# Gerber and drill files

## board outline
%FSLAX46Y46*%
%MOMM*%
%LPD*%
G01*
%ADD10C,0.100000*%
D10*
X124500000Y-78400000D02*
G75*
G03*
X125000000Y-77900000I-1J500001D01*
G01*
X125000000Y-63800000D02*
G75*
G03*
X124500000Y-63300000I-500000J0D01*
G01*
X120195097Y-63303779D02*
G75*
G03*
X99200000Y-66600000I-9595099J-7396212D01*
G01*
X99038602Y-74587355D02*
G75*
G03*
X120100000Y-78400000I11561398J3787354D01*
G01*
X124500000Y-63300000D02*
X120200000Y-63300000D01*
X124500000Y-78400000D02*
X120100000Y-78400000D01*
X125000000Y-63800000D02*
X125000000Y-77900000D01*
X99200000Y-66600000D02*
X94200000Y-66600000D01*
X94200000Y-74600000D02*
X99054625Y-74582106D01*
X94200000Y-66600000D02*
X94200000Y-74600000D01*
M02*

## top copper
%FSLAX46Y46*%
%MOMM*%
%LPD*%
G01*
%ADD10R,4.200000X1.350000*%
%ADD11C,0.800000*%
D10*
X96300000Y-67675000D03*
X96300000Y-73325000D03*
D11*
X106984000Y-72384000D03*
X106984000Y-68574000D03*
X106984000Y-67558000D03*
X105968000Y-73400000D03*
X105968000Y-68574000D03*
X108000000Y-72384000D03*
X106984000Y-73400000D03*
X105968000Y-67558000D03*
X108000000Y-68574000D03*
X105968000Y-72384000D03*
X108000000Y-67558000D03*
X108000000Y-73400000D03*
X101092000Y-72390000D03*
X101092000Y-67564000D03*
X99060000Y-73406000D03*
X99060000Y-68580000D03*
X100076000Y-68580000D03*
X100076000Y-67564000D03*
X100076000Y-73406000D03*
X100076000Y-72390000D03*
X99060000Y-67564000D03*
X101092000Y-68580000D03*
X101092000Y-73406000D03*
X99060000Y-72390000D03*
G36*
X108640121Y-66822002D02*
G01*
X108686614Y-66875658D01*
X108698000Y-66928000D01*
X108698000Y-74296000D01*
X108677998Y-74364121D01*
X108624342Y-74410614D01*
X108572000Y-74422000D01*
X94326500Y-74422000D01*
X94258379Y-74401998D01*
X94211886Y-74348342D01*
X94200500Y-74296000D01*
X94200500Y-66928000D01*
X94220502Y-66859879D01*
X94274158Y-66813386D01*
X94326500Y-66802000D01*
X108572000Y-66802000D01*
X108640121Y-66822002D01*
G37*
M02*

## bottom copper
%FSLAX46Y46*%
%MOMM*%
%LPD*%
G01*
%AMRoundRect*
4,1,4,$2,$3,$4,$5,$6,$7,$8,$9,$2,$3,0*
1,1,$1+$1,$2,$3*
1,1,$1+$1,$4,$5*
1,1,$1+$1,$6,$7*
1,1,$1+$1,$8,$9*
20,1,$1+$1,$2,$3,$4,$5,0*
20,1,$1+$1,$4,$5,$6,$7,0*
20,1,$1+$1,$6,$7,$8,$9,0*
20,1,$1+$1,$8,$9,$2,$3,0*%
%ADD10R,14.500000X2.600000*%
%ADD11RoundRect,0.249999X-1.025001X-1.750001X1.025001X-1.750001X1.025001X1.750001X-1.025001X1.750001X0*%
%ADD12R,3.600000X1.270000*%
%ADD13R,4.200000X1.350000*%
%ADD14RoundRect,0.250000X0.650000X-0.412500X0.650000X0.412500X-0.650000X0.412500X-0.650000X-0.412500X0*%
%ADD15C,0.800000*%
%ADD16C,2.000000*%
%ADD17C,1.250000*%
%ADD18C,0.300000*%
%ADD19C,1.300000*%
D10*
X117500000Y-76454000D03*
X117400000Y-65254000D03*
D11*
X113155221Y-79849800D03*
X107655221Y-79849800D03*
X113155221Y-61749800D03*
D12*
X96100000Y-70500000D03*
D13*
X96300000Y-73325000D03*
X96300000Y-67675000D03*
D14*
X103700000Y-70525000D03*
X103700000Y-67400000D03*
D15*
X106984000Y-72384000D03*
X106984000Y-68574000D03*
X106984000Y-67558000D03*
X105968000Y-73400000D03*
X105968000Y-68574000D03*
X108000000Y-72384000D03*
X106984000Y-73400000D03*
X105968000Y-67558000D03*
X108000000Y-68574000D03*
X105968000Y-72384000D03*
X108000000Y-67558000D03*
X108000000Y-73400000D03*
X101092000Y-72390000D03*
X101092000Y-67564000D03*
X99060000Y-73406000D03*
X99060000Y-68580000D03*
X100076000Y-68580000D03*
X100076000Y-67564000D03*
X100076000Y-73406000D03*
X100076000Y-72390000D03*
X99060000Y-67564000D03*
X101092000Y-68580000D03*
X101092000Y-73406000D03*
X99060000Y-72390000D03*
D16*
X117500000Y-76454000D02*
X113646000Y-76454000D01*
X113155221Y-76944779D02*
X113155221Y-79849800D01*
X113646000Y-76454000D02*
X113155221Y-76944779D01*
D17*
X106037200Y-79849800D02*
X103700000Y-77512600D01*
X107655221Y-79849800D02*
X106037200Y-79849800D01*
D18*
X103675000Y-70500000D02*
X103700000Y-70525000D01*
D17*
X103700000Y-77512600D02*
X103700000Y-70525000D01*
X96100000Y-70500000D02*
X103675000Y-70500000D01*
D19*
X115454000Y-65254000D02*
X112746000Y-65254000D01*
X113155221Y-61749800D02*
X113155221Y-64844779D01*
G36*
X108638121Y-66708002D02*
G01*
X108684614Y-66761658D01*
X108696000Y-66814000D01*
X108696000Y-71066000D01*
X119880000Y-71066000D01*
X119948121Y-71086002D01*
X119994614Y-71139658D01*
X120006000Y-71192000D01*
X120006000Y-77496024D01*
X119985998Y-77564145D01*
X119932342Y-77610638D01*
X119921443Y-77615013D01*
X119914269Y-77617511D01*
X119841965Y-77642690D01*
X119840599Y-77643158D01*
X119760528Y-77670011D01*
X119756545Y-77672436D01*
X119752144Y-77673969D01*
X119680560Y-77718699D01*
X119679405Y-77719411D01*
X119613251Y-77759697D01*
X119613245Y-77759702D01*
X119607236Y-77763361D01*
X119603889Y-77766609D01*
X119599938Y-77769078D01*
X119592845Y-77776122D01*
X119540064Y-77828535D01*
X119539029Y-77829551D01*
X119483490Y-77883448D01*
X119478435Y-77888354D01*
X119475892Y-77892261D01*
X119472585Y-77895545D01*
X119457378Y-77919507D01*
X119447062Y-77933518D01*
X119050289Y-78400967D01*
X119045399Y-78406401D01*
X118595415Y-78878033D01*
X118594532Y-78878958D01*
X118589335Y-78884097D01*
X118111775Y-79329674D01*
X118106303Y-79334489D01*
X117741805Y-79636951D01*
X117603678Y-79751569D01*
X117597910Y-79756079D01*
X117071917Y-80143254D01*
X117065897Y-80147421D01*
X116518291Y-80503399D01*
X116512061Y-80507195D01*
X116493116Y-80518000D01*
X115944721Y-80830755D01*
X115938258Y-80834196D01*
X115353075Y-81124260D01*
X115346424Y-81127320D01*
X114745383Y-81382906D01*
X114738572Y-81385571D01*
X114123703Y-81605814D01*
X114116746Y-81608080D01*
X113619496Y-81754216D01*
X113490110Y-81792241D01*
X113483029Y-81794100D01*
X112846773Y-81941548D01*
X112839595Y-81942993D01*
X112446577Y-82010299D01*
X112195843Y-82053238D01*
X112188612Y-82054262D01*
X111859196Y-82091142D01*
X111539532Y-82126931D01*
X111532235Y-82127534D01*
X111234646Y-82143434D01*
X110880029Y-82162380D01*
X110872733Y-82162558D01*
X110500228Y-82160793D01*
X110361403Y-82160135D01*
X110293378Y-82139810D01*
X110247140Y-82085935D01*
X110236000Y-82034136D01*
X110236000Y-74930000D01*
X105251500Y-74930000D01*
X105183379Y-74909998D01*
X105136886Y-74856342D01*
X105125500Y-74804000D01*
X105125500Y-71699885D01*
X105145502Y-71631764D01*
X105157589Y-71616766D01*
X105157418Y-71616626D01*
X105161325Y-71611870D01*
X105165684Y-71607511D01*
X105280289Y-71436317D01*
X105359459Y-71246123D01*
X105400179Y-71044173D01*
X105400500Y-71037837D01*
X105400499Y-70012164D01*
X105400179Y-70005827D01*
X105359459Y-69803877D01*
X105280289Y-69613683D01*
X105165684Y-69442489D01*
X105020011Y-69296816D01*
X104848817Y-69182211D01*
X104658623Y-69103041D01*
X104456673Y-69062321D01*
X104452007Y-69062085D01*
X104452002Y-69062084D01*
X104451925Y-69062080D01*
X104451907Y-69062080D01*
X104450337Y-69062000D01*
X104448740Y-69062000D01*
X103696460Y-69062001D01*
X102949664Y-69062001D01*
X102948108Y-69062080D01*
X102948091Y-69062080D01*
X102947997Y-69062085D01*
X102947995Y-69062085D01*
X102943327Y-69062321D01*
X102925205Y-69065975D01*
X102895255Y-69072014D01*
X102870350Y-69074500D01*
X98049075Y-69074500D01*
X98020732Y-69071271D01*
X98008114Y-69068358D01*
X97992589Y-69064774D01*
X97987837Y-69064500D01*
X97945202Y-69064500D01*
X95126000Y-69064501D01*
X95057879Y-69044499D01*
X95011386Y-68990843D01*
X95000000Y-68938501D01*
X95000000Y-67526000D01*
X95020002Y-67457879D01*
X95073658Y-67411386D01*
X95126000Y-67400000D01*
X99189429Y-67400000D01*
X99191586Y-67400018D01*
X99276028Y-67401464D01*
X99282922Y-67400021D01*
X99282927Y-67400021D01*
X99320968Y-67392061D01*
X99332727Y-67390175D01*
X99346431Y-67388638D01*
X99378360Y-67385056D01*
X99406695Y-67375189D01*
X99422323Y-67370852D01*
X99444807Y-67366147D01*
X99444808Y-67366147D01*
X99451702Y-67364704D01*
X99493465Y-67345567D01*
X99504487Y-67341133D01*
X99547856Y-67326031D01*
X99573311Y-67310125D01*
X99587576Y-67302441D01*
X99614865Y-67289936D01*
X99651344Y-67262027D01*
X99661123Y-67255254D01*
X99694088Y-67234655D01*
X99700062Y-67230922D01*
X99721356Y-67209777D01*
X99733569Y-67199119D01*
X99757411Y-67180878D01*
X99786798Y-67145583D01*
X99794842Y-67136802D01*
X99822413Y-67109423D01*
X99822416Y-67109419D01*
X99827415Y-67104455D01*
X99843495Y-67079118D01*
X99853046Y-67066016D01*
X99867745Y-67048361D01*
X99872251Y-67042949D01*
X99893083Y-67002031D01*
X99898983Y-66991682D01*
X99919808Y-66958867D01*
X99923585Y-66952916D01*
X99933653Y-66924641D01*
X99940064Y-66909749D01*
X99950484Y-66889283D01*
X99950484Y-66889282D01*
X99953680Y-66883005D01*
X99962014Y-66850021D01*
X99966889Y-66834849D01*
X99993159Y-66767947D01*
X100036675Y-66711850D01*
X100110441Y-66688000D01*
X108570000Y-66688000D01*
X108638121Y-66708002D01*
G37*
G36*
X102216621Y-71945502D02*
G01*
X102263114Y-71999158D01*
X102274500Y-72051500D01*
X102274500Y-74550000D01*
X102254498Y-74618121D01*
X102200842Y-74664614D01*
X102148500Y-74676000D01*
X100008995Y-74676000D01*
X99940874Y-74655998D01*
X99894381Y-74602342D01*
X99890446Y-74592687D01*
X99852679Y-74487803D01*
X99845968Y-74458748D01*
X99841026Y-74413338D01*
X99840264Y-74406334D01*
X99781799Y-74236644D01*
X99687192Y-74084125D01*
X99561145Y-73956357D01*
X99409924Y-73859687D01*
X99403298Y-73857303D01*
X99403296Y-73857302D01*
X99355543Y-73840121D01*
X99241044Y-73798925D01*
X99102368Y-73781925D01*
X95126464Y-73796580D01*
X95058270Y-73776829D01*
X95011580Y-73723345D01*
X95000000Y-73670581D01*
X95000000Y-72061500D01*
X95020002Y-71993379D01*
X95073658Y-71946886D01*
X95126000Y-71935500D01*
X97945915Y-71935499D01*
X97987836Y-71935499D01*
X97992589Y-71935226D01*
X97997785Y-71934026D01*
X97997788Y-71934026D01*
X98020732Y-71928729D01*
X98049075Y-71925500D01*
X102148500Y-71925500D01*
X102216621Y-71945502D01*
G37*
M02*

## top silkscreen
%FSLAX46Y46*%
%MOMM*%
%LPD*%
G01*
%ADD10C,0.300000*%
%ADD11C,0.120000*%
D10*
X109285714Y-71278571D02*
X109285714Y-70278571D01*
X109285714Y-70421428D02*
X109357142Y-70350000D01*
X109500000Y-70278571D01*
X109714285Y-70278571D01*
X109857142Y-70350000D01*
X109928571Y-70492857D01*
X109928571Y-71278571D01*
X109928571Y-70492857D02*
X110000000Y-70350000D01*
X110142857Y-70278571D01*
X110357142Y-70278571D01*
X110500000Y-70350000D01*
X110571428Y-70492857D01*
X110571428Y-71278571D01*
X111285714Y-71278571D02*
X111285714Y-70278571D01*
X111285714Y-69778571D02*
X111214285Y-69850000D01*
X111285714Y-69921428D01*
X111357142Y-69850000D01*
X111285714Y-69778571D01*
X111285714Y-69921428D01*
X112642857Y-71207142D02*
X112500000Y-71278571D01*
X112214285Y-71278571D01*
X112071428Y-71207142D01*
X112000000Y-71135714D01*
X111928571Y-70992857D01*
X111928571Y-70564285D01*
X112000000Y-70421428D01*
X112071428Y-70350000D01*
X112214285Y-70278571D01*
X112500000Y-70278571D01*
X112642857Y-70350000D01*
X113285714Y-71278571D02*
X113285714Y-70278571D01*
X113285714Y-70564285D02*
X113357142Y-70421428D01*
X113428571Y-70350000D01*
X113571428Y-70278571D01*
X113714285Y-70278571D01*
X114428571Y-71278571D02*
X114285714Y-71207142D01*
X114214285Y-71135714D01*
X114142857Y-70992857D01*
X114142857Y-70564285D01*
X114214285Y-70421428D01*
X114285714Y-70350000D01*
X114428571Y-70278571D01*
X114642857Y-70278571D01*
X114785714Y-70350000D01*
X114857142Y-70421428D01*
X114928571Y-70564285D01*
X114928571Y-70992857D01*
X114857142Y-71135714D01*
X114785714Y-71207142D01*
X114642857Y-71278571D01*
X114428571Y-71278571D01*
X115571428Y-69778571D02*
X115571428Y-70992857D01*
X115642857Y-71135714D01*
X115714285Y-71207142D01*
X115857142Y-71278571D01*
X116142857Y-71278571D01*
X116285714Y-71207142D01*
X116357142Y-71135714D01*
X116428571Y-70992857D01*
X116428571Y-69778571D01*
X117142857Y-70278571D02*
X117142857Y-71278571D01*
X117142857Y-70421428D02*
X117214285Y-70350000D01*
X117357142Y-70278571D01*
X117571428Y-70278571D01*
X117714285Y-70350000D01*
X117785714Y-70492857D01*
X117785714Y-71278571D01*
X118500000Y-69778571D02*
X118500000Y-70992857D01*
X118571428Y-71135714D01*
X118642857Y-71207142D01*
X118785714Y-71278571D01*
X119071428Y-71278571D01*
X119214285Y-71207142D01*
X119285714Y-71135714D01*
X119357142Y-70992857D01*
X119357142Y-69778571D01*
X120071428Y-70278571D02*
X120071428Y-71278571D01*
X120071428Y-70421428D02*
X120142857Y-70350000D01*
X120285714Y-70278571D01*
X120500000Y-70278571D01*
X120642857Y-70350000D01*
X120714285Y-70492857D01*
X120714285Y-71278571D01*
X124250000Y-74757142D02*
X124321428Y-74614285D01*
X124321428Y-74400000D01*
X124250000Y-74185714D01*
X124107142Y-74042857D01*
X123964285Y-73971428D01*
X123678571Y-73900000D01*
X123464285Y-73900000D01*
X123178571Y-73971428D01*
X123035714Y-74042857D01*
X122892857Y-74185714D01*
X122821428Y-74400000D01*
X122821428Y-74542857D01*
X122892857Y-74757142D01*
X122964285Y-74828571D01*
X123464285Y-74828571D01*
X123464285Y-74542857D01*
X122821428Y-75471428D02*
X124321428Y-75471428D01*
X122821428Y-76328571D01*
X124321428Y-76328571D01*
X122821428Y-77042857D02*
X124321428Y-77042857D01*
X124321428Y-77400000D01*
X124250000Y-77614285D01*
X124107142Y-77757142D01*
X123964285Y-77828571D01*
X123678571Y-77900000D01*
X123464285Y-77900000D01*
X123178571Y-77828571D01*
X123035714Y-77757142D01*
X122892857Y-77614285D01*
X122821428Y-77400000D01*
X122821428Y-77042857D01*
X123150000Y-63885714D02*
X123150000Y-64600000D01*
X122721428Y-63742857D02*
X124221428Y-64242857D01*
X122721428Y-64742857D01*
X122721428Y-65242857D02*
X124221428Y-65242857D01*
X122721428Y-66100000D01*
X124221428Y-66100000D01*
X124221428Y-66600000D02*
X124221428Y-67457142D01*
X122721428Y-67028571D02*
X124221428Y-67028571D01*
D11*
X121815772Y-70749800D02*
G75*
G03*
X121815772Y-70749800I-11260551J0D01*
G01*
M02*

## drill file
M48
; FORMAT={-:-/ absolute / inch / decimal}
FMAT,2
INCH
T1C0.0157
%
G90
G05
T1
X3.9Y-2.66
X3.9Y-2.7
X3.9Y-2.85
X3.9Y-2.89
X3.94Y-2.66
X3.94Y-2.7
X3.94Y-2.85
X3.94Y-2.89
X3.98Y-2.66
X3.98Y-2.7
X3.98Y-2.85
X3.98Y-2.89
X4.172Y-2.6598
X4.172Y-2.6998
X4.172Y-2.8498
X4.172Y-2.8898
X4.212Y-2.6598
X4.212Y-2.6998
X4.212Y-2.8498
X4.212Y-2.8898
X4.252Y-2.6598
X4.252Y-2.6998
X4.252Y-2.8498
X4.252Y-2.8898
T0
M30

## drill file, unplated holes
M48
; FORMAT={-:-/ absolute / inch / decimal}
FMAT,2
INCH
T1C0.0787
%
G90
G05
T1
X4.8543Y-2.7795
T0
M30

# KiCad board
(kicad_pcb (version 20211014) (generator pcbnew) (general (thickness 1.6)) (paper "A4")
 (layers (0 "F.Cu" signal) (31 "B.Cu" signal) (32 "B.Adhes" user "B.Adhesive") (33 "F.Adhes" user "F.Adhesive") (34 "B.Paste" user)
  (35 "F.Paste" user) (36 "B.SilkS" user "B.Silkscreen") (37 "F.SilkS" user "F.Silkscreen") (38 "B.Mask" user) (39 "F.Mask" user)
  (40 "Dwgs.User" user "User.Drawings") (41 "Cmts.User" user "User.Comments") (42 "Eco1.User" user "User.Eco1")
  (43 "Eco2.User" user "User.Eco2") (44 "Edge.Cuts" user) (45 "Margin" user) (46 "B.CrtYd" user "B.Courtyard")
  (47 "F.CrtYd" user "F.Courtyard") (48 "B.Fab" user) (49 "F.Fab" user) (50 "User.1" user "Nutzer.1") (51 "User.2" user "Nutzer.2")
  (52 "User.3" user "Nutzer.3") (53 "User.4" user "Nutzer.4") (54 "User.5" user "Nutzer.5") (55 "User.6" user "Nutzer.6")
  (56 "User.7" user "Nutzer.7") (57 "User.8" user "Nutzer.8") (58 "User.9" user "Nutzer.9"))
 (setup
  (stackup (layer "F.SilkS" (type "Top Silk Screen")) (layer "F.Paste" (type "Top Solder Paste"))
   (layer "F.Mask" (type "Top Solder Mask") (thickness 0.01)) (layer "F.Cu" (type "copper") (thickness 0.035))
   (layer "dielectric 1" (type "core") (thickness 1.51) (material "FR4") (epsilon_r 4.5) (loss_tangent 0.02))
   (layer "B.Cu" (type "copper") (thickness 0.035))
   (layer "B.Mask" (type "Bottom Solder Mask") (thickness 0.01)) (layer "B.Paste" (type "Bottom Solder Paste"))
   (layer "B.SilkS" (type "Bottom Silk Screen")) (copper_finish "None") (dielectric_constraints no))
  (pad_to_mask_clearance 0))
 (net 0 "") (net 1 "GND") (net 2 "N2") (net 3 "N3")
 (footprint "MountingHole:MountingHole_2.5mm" (layer "F.Cu") (at 123.3 70.6)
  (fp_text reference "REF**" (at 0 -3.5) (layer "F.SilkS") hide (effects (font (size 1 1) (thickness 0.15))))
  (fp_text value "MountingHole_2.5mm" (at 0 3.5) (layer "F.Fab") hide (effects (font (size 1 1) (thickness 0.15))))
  (pad "" np_thru_hole circle (at 0 0) (size 2 2) (drill 2) (layers F&B.Cu *.Mask)))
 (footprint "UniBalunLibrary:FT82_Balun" (layer "F.Cu") (at 110.555221 70.7498)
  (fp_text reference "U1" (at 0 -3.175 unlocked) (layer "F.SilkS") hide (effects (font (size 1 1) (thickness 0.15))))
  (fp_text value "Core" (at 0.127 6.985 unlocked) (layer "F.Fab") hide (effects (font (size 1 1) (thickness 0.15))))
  (fp_circle (center 0 0) (end 6.2 -9.4) (layer "F.SilkS") (width 0.12) (fill none))
  (pad "1" smd roundrect (at 2.6 9.1) (size 2.55 4) (layers "B.Cu" "B.Paste" "B.Mask") (roundrect_rratio 0.09803882353) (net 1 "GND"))
  (pad "2" smd roundrect (at -2.9 9.1) (size 2.55 4) (layers "B.Cu" "B.Paste" "B.Mask") (roundrect_rratio 0.09803882353) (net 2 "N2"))
  (pad "3" smd roundrect (at 2.6 -9) (size 2.55 4) (layers "B.Cu" "B.Paste" "B.Mask") (roundrect_rratio 0.09803882353) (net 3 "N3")))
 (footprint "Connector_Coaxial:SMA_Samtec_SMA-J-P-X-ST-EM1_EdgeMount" (layer "B.Cu") (at 96.3 70.5 90)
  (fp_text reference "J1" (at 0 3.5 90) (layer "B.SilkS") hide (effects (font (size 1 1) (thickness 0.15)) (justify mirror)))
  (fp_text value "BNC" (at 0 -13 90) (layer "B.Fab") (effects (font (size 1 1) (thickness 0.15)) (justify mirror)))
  (pad "1" smd rect (at 0 -0.2 90) (size 1.27 3.6) (layers "B.Cu" "B.Paste" "B.Mask") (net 2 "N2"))
  (pad "2" smd rect (at -2.825 0 90) (size 1.35 4.2) (layers "B.Cu" "B.Paste" "B.Mask") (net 1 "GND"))
  (pad "2" smd rect (at 2.825 0 90) (size 1.35 4.2) (layers "F.Cu" "F.Paste" "F.Mask") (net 1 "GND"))
  (pad "2" smd rect (at -2.825 0 90) (size 1.35 4.2) (layers "F.Cu" "F.Paste" "F.Mask") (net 1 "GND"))
  (pad "2" smd rect (at 2.825 0 90) (size 1.35 4.2) (layers "B.Cu" "B.Paste" "B.Mask") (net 1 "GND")))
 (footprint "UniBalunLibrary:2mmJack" (layer "B.Cu") (at 117.246 76.2 180)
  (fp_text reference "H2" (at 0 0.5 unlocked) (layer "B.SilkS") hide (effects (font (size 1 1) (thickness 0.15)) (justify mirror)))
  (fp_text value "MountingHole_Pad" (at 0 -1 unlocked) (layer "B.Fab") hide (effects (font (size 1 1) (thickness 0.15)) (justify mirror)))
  (pad "1" smd rect (at -0.254 -0.254 180) (size 14.5 2.6) (layers "B.Cu" "B.Paste" "B.Mask") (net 1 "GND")))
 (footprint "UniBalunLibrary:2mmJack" (layer "B.Cu") (at 117.146 65 180)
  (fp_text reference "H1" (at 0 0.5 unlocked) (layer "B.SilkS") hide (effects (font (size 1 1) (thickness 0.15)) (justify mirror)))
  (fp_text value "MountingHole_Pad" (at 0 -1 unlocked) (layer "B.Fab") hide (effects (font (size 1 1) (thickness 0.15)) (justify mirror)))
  (pad "1" smd rect (at -0.254 -0.254 180) (size 14.5 2.6) (layers "B.Cu" "B.Paste" "B.Mask") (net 3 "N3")))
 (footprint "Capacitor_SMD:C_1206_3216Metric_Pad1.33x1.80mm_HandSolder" (layer "B.Cu") (at 103.7 68.9625 90)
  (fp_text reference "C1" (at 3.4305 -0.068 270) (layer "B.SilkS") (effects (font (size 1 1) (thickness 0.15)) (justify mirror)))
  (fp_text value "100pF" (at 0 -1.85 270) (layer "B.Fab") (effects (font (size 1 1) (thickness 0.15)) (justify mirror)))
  (pad "1" smd roundrect (at -1.5625 0 90) (size 1.325 1.8) (layers "B.Cu" "B.Paste" "B.Mask") (roundrect_rratio 0.1886792453) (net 2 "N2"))
  (pad "2" smd roundrect (at 1.5625 0 90) (size 1.325 1.8) (layers "B.Cu" "B.Paste" "B.Mask") (roundrect_rratio 0.1886792453) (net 1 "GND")))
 (gr_line (start 124.5 78.4) (end 120.1 78.4) (layer "Edge.Cuts") (width 0.1))
 (gr_arc (start 125 77.9) (mid 124.853553 78.253553) (end 124.5 78.4) (layer "Edge.Cuts") (width 0.1))
 (gr_arc (start 99.2 66.6) (mid 108.720987 58.731733) (end 120.195097 63.303779) (layer "Edge.Cuts") (width 0.1))
 (gr_arc (start 124.5 63.3) (mid 124.853553 63.446447) (end 125 63.8) (layer "Edge.Cuts") (width 0.1))
 (gr_line (start 124.5 63.3) (end 120.2 63.3) (layer "Edge.Cuts") (width 0.1))
 (gr_line (start 99.2 66.6) (end 94.2 66.6) (layer "Edge.Cuts") (width 0.1))
 (gr_line (start 94.2 74.6) (end 99.054625 74.582106) (layer "Edge.Cuts") (width 0.1))
 (gr_line (start 125 63.8) (end 125 77.9) (layer "Edge.Cuts") (width 0.1))
 (gr_line (start 94.2 66.6) (end 94.2 74.6) (layer "Edge.Cuts") (width 0.1))
 (gr_arc (start 120.1 78.4) (mid 108.432881 82.771366) (end 99.038602 74.587355) (layer "Edge.Cuts") (width 0.1))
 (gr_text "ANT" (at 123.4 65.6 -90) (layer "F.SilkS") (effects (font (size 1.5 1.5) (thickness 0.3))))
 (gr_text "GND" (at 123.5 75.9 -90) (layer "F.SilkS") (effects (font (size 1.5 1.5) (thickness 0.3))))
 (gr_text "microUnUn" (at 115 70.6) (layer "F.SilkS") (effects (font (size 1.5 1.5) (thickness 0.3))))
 (segment (start 106.0372 79.8498) (end 103.7 77.5126) (width 1.25) (layer "B.Cu") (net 2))
 (segment (start 107.655221 79.8498) (end 106.0372 79.8498) (width 1.25) (layer "B.Cu") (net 2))
 (segment (start 103.675 70.5) (end 103.7 70.525) (width 0.3) (layer "B.Cu") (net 2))
 (segment (start 103.7 77.5126) (end 103.7 70.525) (width 1.25) (layer "B.Cu") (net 2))
 (segment (start 96.1 70.5) (end 103.675 70.5) (width 1.25) (layer "B.Cu") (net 2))
 (via (at 105.968 73.4) (size 0.8) (drill 0.4) (layers "F.Cu" "B.Cu") (free) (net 1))
 (via (at 108 73.4) (size 0.8) (drill 0.4) (layers "F.Cu" "B.Cu") (free) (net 1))
 (via (at 101.092 72.39) (size 0.8) (drill 0.4) (layers "F.Cu" "B.Cu") (free) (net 1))
 (via (at 105.968 67.558) (size 0.8) (drill 0.4) (layers "F.Cu" "B.Cu") (free) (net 1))
 (via (at 101.092 67.564) (size 0.8) (drill 0.4) (layers "F.Cu" "B.Cu") (free) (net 1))
 (via (at 99.06 73.406) (size 0.8) (drill 0.4) (layers "F.Cu" "B.Cu") (free) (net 1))
 (via (at 99.06 68.58) (size 0.8) (drill 0.4) (layers "F.Cu" "B.Cu") (free) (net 1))
 (via (at 100.076 68.58) (size 0.8) (drill 0.4) (layers "F.Cu" "B.Cu") (free) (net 1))
 (via (at 100.076 67.564) (size 0.8) (drill 0.4) (layers "F.Cu" "B.Cu") (free) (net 1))
 (via (at 100.076 73.406) (size 0.8) (drill 0.4) (layers "F.Cu" "B.Cu") (free) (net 1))
 (via (at 100.076 72.39) (size 0.8) (drill 0.4) (layers "F.Cu" "B.Cu") (free) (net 1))
 (via (at 106.984 68.574) (size 0.8) (drill 0.4) (layers "F.Cu" "B.Cu") (free) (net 1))
 (via (at 108 67.558) (size 0.8) (drill 0.4) (layers "F.Cu" "B.Cu") (free) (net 1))
 (via (at 105.968 72.384) (size 0.8) (drill 0.4) (layers "F.Cu" "B.Cu") (free) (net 1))
 (via (at 99.06 67.564) (size 0.8) (drill 0.4) (layers "F.Cu" "B.Cu") (free) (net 1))
 (via (at 108 72.384) (size 0.8) (drill 0.4) (layers "F.Cu" "B.Cu") (free) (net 1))
 (via (at 108 68.574) (size 0.8) (drill 0.4) (layers "F.Cu" "B.Cu") (free) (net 1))
 (via (at 106.984 67.558) (size 0.8) (drill 0.4) (layers "F.Cu" "B.Cu") (free) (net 1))
 (via (at 106.984 73.4) (size 0.8) (drill 0.4) (layers "F.Cu" "B.Cu") (free) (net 1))
 (via (at 101.092 68.58) (size 0.8) (drill 0.4) (layers "F.Cu" "B.Cu") (free) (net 1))
 (via (at 106.984 72.384) (size 0.8) (drill 0.4) (layers "F.Cu" "B.Cu") (free) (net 1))
 (via (at 101.092 73.406) (size 0.8) (drill 0.4) (layers "F.Cu" "B.Cu") (free) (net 1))
 (via (at 99.06 72.39) (size 0.8) (drill 0.4) (layers "F.Cu" "B.Cu") (free) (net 1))
 (via (at 105.968 68.574) (size 0.8) (drill 0.4) (layers "F.Cu" "B.Cu") (free) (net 1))
 (segment (start 117.5 76.454) (end 113.646 76.454) (width 2) (layer "B.Cu") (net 1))
 (segment (start 113.155221 76.944779) (end 113.155221 79.8498) (width 2) (layer "B.Cu") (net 1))
 (segment (start 113.646 76.454) (end 113.155221 76.944779) (width 2) (layer "B.Cu") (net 1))
 (segment (start 115.454 65.254) (end 112.746 65.254) (width 1.3) (layer "B.Cu") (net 3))
 (segment (start 113.155221 61.7498) (end 113.155221 64.844779) (width 1.3) (layer "B.Cu") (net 3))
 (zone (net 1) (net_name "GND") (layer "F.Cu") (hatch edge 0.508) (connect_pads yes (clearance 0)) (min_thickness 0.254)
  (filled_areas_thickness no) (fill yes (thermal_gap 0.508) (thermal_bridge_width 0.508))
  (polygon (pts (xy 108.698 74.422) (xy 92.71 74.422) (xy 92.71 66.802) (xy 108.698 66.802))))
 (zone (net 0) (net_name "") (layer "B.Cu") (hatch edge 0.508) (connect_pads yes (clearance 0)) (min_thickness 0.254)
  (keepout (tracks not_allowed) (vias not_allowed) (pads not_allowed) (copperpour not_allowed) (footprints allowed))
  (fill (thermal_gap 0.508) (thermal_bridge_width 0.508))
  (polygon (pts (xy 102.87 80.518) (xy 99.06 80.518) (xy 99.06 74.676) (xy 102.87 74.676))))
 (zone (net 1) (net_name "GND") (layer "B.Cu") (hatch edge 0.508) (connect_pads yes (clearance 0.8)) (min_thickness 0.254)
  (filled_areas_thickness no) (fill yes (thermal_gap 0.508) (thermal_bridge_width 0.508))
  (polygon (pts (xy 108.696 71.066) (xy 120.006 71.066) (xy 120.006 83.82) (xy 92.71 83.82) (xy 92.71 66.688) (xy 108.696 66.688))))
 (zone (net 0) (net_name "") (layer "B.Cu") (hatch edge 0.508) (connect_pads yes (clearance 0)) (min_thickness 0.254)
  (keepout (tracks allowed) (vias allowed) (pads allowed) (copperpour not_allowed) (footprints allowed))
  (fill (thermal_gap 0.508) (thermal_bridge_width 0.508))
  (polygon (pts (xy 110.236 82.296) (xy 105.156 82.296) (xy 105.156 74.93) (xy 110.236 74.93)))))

